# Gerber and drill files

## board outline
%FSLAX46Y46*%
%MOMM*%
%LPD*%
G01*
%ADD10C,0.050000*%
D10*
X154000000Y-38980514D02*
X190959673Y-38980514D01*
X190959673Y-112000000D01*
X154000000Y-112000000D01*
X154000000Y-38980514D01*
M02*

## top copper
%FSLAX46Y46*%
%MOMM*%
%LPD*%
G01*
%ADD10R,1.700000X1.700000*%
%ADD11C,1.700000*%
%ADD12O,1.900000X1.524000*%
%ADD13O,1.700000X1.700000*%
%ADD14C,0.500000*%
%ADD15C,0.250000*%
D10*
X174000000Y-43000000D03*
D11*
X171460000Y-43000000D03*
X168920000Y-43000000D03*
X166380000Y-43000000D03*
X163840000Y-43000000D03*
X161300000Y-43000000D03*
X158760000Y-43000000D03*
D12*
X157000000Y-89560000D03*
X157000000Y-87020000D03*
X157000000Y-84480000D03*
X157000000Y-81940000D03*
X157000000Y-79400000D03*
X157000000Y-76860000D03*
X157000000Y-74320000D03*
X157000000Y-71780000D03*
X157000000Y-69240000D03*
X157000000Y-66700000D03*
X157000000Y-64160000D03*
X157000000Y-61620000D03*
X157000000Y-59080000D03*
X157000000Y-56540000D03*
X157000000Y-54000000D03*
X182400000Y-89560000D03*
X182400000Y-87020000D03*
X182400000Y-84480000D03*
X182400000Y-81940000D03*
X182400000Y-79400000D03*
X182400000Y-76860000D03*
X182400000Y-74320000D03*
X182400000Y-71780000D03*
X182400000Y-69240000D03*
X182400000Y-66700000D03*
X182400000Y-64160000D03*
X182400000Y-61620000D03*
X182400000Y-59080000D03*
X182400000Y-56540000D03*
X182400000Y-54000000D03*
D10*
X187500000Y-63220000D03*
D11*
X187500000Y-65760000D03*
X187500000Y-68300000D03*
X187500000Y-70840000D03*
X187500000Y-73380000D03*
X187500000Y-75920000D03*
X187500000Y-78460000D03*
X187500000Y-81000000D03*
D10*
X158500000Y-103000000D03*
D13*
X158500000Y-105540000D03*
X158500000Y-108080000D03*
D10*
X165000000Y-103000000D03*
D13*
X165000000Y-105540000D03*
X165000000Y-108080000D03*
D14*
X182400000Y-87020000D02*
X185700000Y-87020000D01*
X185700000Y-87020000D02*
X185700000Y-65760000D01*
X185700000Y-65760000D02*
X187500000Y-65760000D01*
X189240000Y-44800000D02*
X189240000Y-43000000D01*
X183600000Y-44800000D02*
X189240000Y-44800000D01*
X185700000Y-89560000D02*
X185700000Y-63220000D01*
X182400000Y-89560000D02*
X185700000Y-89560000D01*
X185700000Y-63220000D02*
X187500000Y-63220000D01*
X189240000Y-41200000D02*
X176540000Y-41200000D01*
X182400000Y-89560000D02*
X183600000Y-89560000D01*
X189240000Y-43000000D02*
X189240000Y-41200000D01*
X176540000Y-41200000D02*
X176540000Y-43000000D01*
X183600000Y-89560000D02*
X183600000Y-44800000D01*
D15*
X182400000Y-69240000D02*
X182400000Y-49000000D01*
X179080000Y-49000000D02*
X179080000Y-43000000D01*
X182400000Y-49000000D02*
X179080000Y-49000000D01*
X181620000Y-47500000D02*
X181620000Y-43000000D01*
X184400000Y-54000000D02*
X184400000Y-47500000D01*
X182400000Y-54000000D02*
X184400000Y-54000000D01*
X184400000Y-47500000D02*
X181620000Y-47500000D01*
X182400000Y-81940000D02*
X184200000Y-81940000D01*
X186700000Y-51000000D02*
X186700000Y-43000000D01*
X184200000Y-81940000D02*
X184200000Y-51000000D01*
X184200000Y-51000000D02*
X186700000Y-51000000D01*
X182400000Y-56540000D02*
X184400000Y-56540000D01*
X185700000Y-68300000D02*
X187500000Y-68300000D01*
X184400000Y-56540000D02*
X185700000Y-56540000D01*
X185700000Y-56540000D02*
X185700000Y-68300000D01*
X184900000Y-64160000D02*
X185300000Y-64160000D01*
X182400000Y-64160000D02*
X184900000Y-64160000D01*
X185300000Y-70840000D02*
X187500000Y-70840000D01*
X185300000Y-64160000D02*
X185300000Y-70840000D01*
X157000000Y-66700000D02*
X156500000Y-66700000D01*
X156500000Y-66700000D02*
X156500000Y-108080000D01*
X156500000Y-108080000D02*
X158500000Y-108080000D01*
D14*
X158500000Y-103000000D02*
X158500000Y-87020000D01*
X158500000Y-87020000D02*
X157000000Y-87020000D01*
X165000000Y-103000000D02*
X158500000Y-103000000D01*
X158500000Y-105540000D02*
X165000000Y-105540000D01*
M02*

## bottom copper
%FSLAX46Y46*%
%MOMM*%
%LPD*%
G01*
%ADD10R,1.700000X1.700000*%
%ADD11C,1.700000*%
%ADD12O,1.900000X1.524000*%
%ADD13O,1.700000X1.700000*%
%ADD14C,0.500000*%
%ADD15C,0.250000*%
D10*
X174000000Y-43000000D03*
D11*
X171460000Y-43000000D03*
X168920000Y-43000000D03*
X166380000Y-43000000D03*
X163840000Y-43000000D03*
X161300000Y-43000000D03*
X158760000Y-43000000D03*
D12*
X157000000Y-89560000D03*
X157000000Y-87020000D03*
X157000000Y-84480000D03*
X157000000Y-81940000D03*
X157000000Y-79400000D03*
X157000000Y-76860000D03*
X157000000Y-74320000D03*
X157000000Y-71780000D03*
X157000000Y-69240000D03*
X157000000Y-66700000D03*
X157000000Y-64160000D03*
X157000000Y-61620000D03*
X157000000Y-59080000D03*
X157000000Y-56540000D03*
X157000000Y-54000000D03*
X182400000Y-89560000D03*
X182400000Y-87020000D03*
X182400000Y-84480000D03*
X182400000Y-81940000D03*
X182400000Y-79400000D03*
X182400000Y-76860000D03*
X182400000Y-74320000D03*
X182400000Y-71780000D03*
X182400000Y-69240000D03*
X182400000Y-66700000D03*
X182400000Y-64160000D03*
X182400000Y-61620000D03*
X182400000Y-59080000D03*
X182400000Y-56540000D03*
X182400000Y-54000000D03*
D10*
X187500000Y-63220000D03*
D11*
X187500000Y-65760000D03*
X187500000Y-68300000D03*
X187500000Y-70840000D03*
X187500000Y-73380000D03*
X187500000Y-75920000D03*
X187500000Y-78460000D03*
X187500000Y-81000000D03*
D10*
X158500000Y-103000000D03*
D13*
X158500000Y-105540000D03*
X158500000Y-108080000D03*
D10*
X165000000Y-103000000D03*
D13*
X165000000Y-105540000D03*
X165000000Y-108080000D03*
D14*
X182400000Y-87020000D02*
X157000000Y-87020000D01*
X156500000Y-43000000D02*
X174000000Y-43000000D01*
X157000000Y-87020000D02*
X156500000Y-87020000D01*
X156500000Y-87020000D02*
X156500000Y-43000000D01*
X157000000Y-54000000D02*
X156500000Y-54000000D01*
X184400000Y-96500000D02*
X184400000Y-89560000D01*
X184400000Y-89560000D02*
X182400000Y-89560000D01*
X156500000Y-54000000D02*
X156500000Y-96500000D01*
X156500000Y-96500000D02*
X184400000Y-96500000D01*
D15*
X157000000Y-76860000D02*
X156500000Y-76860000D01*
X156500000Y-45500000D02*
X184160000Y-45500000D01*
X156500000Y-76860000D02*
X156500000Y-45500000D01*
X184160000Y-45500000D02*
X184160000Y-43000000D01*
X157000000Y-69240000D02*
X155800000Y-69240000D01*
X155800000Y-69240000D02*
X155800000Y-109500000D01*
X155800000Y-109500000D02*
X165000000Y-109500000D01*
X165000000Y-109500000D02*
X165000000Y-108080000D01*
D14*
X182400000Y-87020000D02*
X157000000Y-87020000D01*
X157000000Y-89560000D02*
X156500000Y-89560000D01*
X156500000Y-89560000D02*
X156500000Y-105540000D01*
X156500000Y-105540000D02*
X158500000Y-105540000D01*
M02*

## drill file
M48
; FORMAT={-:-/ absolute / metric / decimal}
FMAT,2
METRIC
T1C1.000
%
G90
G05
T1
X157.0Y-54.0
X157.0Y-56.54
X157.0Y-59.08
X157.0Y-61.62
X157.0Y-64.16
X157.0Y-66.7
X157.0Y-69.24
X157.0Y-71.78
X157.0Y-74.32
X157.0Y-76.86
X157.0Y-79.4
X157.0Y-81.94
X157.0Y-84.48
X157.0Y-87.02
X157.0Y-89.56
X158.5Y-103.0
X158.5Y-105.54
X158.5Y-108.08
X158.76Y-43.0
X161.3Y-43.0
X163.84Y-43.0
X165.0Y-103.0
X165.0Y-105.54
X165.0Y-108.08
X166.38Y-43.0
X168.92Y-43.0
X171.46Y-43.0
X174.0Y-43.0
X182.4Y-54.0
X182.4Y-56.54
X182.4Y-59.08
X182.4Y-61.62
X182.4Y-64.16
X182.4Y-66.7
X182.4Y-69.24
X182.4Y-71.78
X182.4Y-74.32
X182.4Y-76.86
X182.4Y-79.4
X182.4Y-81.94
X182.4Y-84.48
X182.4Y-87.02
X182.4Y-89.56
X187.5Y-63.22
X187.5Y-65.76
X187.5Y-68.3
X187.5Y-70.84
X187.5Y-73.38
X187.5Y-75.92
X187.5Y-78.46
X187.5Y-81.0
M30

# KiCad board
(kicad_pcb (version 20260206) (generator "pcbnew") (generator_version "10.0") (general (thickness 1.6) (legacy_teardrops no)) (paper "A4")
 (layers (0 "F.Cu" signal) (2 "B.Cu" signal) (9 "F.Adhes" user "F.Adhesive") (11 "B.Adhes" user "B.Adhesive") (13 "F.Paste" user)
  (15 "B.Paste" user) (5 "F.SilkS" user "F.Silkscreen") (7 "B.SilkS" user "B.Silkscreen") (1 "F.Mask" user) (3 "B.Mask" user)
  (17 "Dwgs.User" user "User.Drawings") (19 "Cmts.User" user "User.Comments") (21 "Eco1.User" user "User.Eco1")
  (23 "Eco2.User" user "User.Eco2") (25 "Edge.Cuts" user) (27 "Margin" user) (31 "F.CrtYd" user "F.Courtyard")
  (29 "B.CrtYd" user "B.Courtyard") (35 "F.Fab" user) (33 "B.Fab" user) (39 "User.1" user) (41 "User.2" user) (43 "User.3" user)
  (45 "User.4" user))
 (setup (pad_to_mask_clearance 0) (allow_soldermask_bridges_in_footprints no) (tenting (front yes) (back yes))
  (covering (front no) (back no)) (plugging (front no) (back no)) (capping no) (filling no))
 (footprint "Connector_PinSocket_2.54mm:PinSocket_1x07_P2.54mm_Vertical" (layer "F.Cu") (at 174 43 -90)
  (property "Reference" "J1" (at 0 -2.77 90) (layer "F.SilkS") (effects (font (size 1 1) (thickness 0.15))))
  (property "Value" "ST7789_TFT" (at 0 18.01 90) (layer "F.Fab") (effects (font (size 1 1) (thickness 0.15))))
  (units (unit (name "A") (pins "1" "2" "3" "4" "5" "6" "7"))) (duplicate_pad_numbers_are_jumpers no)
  (pad "1" thru_hole rect (at 0 0 270) (size 1.7 1.7) (drill 1) (layers "*.Cu" "*.Mask") (remove_unused_layers no) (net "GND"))
  (pad "2" thru_hole circle (at 0 2.54 270) (size 1.7 1.7) (drill 1) (layers "*.Cu" "*.Mask") (remove_unused_layers no) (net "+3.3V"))
  (pad "3" thru_hole circle (at 0 5.08 270) (size 1.7 1.7) (drill 1) (layers "*.Cu" "*.Mask") (remove_unused_layers no) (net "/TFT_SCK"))
  (pad "4" thru_hole circle (at 0 7.62 270) (size 1.7 1.7) (drill 1) (layers "*.Cu" "*.Mask") (remove_unused_layers no) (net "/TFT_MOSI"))
  (pad "5" thru_hole circle (at 0 10.16 270) (size 1.7 1.7) (drill 1) (layers "*.Cu" "*.Mask") (remove_unused_layers no) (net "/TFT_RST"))
  (pad "6" thru_hole circle (at 0 12.7 270) (size 1.7 1.7) (drill 1) (layers "*.Cu" "*.Mask") (remove_unused_layers no) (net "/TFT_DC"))
  (pad "7" thru_hole circle (at 0 15.24 270) (size 1.7 1.7) (drill 1) (layers "*.Cu" "*.Mask") (remove_unused_layers no) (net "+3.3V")))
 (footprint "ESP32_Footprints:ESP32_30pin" (layer "F.Cu") (at 168.92754 72.540187)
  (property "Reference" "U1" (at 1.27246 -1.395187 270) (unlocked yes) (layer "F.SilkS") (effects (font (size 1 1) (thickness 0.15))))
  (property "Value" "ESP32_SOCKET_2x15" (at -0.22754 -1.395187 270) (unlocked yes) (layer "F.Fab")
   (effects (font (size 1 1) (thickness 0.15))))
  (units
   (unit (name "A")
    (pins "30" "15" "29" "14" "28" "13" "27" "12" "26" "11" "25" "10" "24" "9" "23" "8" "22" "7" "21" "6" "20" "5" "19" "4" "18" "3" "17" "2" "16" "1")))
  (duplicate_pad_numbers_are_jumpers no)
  (pad "1" thru_hole oval (at -11.92754 17.019813 270) (size 1.524 1.9) (drill 1) (layers "*.Cu" "*.Mask") (remove_unused_layers no)
   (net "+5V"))
  (pad "2" thru_hole oval (at -11.92754 14.479813 270) (size 1.524 1.9) (drill 1) (layers "*.Cu" "*.Mask") (remove_unused_layers no)
   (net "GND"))
  (pad "3" thru_hole oval (at -11.92754 11.939813 270) (size 1.524 1.9) (drill 1) (layers "*.Cu" "*.Mask") (remove_unused_layers no)
   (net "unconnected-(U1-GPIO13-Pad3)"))
  (pad "4" thru_hole oval (at -11.92754 9.399813 270) (size 1.524 1.9) (drill 1) (layers "*.Cu" "*.Mask") (remove_unused_layers no)
   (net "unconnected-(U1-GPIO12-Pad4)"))
  (pad "5" thru_hole oval (at -11.92754 6.859813 270) (size 1.524 1.9) (drill 1) (layers "*.Cu" "*.Mask") (remove_unused_layers no)
   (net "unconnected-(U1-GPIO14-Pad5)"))
  (pad "6" thru_hole oval (at -11.92754 4.319813 270) (size 1.524 1.9) (drill 1) (layers "*.Cu" "*.Mask") (remove_unused_layers no)
   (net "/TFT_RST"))
  (pad "7" thru_hole oval (at -11.92754 1.779813 270) (size 1.524 1.9) (drill 1) (layers "*.Cu" "*.Mask") (remove_unused_layers no)
   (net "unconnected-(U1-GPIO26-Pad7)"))
  (pad "8" thru_hole oval (at -11.92754 -0.760187 270) (size 1.524 1.9) (drill 1) (layers "*.Cu" "*.Mask") (remove_unused_layers no)
   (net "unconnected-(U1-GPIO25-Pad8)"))
  (pad "9" thru_hole oval (at -11.92754 -3.300187 270) (size 1.524 1.9) (drill 1) (layers "*.Cu" "*.Mask") (remove_unused_layers no)
   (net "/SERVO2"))
  (pad "10" thru_hole oval (at -11.92754 -5.840187 270) (size 1.524 1.9) (drill 1) (layers "*.Cu" "*.Mask") (remove_unused_layers no)
   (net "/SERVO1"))
  (pad "11" thru_hole oval (at -11.92754 -8.380187 270) (size 1.524 1.9) (drill 1) (layers "*.Cu" "*.Mask") (remove_unused_layers no)
   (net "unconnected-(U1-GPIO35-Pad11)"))
  (pad "12" thru_hole oval (at -11.92754 -10.920187 270) (size 1.524 1.9) (drill 1) (layers "*.Cu" "*.Mask") (remove_unused_layers no)
   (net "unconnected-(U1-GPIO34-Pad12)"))
  (pad "13" thru_hole oval (at -11.92754 -13.460187 270) (size 1.524 1.9) (drill 1) (layers "*.Cu" "*.Mask") (remove_unused_layers no)
   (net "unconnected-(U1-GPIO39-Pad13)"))
  (pad "14" thru_hole oval (at -11.92754 -16.000187 270) (size 1.524 1.9) (drill 1) (layers "*.Cu" "*.Mask") (remove_unused_layers no)
   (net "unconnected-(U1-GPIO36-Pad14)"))
  (pad "15" thru_hole oval (at -11.92754 -18.540187 270) (size 1.524 1.9) (drill 1) (layers "*.Cu" "*.Mask") (remove_unused_layers no)
   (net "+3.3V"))
  (pad "16" thru_hole oval (at 13.47246 17.019813 270) (size 1.524 1.9) (drill 1) (layers "*.Cu" "*.Mask") (remove_unused_layers no)
   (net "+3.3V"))
  (pad "17" thru_hole oval (at 13.47246 14.479813 270) (size 1.524 1.9) (drill 1) (layers "*.Cu" "*.Mask") (remove_unused_layers no)
   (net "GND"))
  (pad "18" thru_hole oval (at 13.47246 11.939813 270) (size 1.524 1.9) (drill 1) (layers "*.Cu" "*.Mask") (remove_unused_layers no)
   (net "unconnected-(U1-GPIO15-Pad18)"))
  (pad "19" thru_hole oval (at 13.47246 9.399813 270) (size 1.524 1.9) (drill 1) (layers "*.Cu" "*.Mask") (remove_unused_layers no)
   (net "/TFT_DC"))
  (pad "20" thru_hole oval (at 13.47246 6.859813 270) (size 1.524 1.9) (drill 1) (layers "*.Cu" "*.Mask" "Dwgs.User")
   (remove_unused_layers no) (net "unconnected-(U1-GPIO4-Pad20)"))
  (pad "21" thru_hole oval (at 13.47246 4.319813 270) (size 1.524 1.9) (drill 1) (layers "*.Cu" "*.Mask") (remove_unused_layers no)
   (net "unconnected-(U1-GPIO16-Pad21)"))
  (pad "22" thru_hole oval (at 13.47246 1.779813 270) (size 1.524 1.9) (drill 1) (layers "*.Cu" "*.Mask") (remove_unused_layers no)
   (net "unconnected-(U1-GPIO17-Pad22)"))
  (pad "23" thru_hole oval (at 13.47246 -0.760187 270) (size 1.524 1.9) (drill 1) (layers "*.Cu" "*.Mask") (remove_unused_layers no)
   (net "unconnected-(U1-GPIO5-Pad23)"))
  (pad "24" thru_hole oval (at 13.47246 -3.300187 270) (size 1.524 1.9) (drill 1) (layers "*.Cu" "*.Mask") (remove_unused_layers no)
   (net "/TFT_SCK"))
  (pad "25" thru_hole oval (at 13.47246 -5.840187 270) (size 1.524 1.9) (drill 1) (layers "*.Cu" "*.Mask") (remove_unused_layers no)
   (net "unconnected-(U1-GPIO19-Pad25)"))
  (pad "26" thru_hole oval (at 13.47246 -8.380187 270) (size 1.524 1.9) (drill 1) (layers "*.Cu" "*.Mask") (remove_unused_layers no)
   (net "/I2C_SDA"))
  (pad "27" thru_hole oval (at 13.47246 -10.920187 270) (size 1.524 1.9) (drill 1) (layers "*.Cu" "*.Mask") (remove_unused_layers no)
   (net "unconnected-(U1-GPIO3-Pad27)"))
  (pad "28" thru_hole oval (at 13.47246 -13.460187 270) (size 1.524 1.9) (drill 1) (layers "*.Cu" "*.Mask") (remove_unused_layers no)
   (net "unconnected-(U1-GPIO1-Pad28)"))
  (pad "29" thru_hole oval (at 13.47246 -16.000187 270) (size 1.524 1.9) (drill 1) (layers "*.Cu" "*.Mask") (remove_unused_layers no)
   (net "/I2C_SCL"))
  (pad "30" thru_hole oval (at 13.47246 -18.540187 270) (size 1.524 1.9) (drill 1) (layers "*.Cu" "*.Mask") (remove_unused_layers no)
   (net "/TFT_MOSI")))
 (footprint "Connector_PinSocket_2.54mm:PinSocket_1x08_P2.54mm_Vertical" (layer "F.Cu") (at 187.5 63.22)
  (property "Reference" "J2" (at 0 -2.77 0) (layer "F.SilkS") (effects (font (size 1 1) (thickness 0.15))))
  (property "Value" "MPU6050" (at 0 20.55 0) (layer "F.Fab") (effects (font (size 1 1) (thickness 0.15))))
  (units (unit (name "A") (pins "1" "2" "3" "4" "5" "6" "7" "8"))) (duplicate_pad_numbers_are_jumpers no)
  (pad "1" thru_hole rect (at 0 0) (size 1.7 1.7) (drill 1) (layers "*.Cu" "*.Mask") (remove_unused_layers no) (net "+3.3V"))
  (pad "2" thru_hole circle (at 0 2.54) (size 1.7 1.7) (drill 1) (layers "*.Cu" "*.Mask") (remove_unused_layers no) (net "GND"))
  (pad "3" thru_hole circle (at 0 5.08) (size 1.7 1.7) (drill 1) (layers "*.Cu" "*.Mask") (remove_unused_layers no) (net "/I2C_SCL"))
  (pad "4" thru_hole circle (at 0 7.62) (size 1.7 1.7) (drill 1) (layers "*.Cu" "*.Mask") (remove_unused_layers no) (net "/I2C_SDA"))
  (pad "5" thru_hole circle (at 0 10.16) (size 1.7 1.7) (drill 1) (layers "*.Cu" "*.Mask") (remove_unused_layers no)
   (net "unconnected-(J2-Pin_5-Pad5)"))
  (pad "6" thru_hole circle (at 0 12.7) (size 1.7 1.7) (drill 1) (layers "*.Cu" "*.Mask") (remove_unused_layers no)
   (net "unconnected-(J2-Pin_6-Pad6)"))
  (pad "7" thru_hole circle (at 0 15.24) (size 1.7 1.7) (drill 1) (layers "*.Cu" "*.Mask") (remove_unused_layers no)
   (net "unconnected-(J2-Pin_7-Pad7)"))
  (pad "8" thru_hole circle (at 0 17.78) (size 1.7 1.7) (drill 1) (layers "*.Cu" "*.Mask") (remove_unused_layers no)
   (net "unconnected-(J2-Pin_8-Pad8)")))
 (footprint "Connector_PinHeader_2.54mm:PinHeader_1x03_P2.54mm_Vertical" (layer "F.Cu") (at 158.5 103)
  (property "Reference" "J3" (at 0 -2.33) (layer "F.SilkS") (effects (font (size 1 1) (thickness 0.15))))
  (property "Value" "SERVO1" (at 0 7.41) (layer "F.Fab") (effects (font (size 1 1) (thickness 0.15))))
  (pad "1" thru_hole rect (at 0 0) (size 1.7 1.7) (drill 1) (layers "*.Cu" "*.Mask") (remove_unused_layers no) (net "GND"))
  (pad "2" thru_hole oval (at 0 2.54) (size 1.7 1.7) (drill 1) (layers "*.Cu" "*.Mask") (remove_unused_layers no) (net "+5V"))
  (pad "3" thru_hole oval (at 0 5.08) (size 1.7 1.7) (drill 1) (layers "*.Cu" "*.Mask") (remove_unused_layers no) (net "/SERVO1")))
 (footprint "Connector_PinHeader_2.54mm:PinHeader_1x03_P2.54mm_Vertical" (layer "F.Cu") (at 165 103)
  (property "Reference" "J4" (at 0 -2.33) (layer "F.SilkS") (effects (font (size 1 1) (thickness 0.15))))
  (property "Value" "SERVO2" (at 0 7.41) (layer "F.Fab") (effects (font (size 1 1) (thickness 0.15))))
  (pad "1" thru_hole rect (at 0 0) (size 1.7 1.7) (drill 1) (layers "*.Cu" "*.Mask") (remove_unused_layers no) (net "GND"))
  (pad "2" thru_hole oval (at 0 2.54) (size 1.7 1.7) (drill 1) (layers "*.Cu" "*.Mask") (remove_unused_layers no) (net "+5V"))
  (pad "3" thru_hole oval (at 0 5.08) (size 1.7 1.7) (drill 1) (layers "*.Cu" "*.Mask") (remove_unused_layers no) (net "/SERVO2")))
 (gr_rect (start 154 38.980514) (end 190.959673 112) (stroke (width 0.05) (type default)) (fill no) (layer "Edge.Cuts"))
 (segment (start 182.4 87.02) (end 185.7 87.02) (width 0.5) (layer "F.Cu") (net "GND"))
 (segment (start 185.7 87.02) (end 185.7 65.76) (width 0.5) (layer "F.Cu") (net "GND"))
 (segment (start 185.7 65.76) (end 187.5 65.76) (width 0.5) (layer "F.Cu") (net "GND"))
 (segment (start 182.4 87.02) (end 157 87.02) (width 0.5) (layer "B.Cu") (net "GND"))
 (segment (start 156.5 43) (end 174 43) (width 0.5) (layer "B.Cu") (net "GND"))
 (segment (start 157 87.02) (end 156.5 87.02) (width 0.5) (layer "B.Cu") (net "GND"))
 (segment (start 156.5 87.02) (end 156.5 43) (width 0.5) (layer "B.Cu") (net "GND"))
 (segment (start 189.24 44.8) (end 189.24 43) (width 0.5) (layer "F.Cu") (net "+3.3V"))
 (segment (start 183.6 44.8) (end 189.24 44.8) (width 0.5) (layer "F.Cu") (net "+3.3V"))
 (segment (start 185.7 89.56) (end 185.7 63.22) (width 0.5) (layer "F.Cu") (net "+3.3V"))
 (segment (start 182.4 89.56) (end 185.7 89.56) (width 0.5) (layer "F.Cu") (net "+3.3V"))
 (segment (start 185.7 63.22) (end 187.5 63.22) (width 0.5) (layer "F.Cu") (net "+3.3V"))
 (segment (start 189.24 41.2) (end 176.54 41.2) (width 0.5) (layer "F.Cu") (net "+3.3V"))
 (segment (start 182.4 89.56) (end 183.6 89.56) (width 0.5) (layer "F.Cu") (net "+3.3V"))
 (segment (start 189.24 43) (end 189.24 41.2) (width 0.5) (layer "F.Cu") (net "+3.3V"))
 (segment (start 176.54 41.2) (end 176.54 43) (width 0.5) (layer "F.Cu") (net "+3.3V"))
 (segment (start 183.6 89.56) (end 183.6 44.8) (width 0.5) (layer "F.Cu") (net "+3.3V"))
 (segment (start 157 54) (end 156.5 54) (width 0.5) (layer "B.Cu") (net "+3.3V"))
 (segment (start 184.4 96.5) (end 184.4 89.56) (width 0.5) (layer "B.Cu") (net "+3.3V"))
 (segment (start 184.4 89.56) (end 182.4 89.56) (width 0.5) (layer "B.Cu") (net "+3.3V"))
 (segment (start 156.5 54) (end 156.5 96.5) (width 0.5) (layer "B.Cu") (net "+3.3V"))
 (segment (start 156.5 96.5) (end 184.4 96.5) (width 0.5) (layer "B.Cu") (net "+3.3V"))
 (segment (start 182.4 69.24) (end 182.4 49) (width 0.25) (layer "F.Cu") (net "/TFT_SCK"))
 (segment (start 179.08 49) (end 179.08 43) (width 0.25) (layer "F.Cu") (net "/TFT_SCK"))
 (segment (start 182.4 49) (end 179.08 49) (width 0.25) (layer "F.Cu") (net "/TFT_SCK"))
 (segment (start 181.62 47.5) (end 181.62 43) (width 0.25) (layer "F.Cu") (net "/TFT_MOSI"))
 (segment (start 184.4 54) (end 184.4 47.5) (width 0.25) (layer "F.Cu") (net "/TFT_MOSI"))
 (segment (start 182.4 54) (end 184.4 54) (width 0.25) (layer "F.Cu") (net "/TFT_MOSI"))
 (segment (start 184.4 47.5) (end 181.62 47.5) (width 0.25) (layer "F.Cu") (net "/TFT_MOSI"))
 (segment (start 157 76.86) (end 156.5 76.86) (width 0.25) (layer "B.Cu") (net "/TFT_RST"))
 (segment (start 156.5 45.5) (end 184.16 45.5) (width 0.25) (layer "B.Cu") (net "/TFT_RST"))
 (segment (start 156.5 76.86) (end 156.5 45.5) (width 0.25) (layer "B.Cu") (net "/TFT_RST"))
 (segment (start 184.16 45.5) (end 184.16 43) (width 0.25) (layer "B.Cu") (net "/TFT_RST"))
 (segment (start 182.4 81.94) (end 184.2 81.94) (width 0.25) (layer "F.Cu") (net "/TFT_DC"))
 (segment (start 186.7 51) (end 186.7 43) (width 0.25) (layer "F.Cu") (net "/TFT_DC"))
 (segment (start 184.2 81.94) (end 184.2 51) (width 0.25) (layer "F.Cu") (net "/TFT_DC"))
 (segment (start 184.2 51) (end 186.7 51) (width 0.25) (layer "F.Cu") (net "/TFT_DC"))
 (segment (start 182.4 56.54) (end 184.4 56.54) (width 0.25) (layer "F.Cu") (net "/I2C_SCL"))
 (segment (start 185.7 68.3) (end 187.5 68.3) (width 0.25) (layer "F.Cu") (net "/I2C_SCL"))
 (segment (start 184.4 56.54) (end 185.7 56.54) (width 0.25) (layer "F.Cu") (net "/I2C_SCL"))
 (segment (start 185.7 56.54) (end 185.7 68.3) (width 0.25) (layer "F.Cu") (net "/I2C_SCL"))
 (segment (start 184.9 64.16) (end 185.3 64.16) (width 0.25) (layer "F.Cu") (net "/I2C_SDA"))
 (segment (start 182.4 64.16) (end 184.9 64.16) (width 0.25) (layer "F.Cu") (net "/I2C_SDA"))
 (segment (start 185.3 70.84) (end 187.5 70.84) (width 0.25) (layer "F.Cu") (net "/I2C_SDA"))
 (segment (start 185.3 64.16) (end 185.3 70.84) (width 0.25) (layer "F.Cu") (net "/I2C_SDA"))
 (segment (start 157 66.7) (end 156.5 66.7) (width 0.25) (layer "F.Cu") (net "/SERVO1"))
 (segment (start 156.5 66.7) (end 156.5 108.08) (width 0.25) (layer "F.Cu") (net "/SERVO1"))
 (segment (start 156.5 108.08) (end 158.5 108.08) (width 0.25) (layer "F.Cu") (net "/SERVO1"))
 (segment (start 157 69.24) (end 155.8 69.24) (width 0.25) (layer "B.Cu") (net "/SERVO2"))
 (segment (start 155.8 69.24) (end 155.8 109.5) (width 0.25) (layer "B.Cu") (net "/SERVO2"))
 (segment (start 155.8 109.5) (end 165 109.5) (width 0.25) (layer "B.Cu") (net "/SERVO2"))
 (segment (start 165 109.5) (end 165 108.08) (width 0.25) (layer "B.Cu") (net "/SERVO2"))
 (segment (start 158.5 103) (end 158.5 87.02) (width 0.5) (layer "F.Cu") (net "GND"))
 (segment (start 158.5 87.02) (end 157 87.02) (width 0.5) (layer "F.Cu") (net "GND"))
 (segment (start 165 103) (end 158.5 103) (width 0.5) (layer "F.Cu") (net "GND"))
 (segment (start 182.4 87.02) (end 157 87.02) (width 0.5) (layer "B.Cu") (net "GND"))
 (segment (start 157 89.56) (end 156.5 89.56) (width 0.5) (layer "B.Cu") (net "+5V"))
 (segment (start 156.5 89.56) (end 156.5 105.54) (width 0.5) (layer "B.Cu") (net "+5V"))
 (segment (start 156.5 105.54) (end 158.5 105.54) (width 0.5) (layer "B.Cu") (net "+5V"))
 (segment (start 158.5 105.54) (end 165 105.54) (width 0.5) (layer "F.Cu") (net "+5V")))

